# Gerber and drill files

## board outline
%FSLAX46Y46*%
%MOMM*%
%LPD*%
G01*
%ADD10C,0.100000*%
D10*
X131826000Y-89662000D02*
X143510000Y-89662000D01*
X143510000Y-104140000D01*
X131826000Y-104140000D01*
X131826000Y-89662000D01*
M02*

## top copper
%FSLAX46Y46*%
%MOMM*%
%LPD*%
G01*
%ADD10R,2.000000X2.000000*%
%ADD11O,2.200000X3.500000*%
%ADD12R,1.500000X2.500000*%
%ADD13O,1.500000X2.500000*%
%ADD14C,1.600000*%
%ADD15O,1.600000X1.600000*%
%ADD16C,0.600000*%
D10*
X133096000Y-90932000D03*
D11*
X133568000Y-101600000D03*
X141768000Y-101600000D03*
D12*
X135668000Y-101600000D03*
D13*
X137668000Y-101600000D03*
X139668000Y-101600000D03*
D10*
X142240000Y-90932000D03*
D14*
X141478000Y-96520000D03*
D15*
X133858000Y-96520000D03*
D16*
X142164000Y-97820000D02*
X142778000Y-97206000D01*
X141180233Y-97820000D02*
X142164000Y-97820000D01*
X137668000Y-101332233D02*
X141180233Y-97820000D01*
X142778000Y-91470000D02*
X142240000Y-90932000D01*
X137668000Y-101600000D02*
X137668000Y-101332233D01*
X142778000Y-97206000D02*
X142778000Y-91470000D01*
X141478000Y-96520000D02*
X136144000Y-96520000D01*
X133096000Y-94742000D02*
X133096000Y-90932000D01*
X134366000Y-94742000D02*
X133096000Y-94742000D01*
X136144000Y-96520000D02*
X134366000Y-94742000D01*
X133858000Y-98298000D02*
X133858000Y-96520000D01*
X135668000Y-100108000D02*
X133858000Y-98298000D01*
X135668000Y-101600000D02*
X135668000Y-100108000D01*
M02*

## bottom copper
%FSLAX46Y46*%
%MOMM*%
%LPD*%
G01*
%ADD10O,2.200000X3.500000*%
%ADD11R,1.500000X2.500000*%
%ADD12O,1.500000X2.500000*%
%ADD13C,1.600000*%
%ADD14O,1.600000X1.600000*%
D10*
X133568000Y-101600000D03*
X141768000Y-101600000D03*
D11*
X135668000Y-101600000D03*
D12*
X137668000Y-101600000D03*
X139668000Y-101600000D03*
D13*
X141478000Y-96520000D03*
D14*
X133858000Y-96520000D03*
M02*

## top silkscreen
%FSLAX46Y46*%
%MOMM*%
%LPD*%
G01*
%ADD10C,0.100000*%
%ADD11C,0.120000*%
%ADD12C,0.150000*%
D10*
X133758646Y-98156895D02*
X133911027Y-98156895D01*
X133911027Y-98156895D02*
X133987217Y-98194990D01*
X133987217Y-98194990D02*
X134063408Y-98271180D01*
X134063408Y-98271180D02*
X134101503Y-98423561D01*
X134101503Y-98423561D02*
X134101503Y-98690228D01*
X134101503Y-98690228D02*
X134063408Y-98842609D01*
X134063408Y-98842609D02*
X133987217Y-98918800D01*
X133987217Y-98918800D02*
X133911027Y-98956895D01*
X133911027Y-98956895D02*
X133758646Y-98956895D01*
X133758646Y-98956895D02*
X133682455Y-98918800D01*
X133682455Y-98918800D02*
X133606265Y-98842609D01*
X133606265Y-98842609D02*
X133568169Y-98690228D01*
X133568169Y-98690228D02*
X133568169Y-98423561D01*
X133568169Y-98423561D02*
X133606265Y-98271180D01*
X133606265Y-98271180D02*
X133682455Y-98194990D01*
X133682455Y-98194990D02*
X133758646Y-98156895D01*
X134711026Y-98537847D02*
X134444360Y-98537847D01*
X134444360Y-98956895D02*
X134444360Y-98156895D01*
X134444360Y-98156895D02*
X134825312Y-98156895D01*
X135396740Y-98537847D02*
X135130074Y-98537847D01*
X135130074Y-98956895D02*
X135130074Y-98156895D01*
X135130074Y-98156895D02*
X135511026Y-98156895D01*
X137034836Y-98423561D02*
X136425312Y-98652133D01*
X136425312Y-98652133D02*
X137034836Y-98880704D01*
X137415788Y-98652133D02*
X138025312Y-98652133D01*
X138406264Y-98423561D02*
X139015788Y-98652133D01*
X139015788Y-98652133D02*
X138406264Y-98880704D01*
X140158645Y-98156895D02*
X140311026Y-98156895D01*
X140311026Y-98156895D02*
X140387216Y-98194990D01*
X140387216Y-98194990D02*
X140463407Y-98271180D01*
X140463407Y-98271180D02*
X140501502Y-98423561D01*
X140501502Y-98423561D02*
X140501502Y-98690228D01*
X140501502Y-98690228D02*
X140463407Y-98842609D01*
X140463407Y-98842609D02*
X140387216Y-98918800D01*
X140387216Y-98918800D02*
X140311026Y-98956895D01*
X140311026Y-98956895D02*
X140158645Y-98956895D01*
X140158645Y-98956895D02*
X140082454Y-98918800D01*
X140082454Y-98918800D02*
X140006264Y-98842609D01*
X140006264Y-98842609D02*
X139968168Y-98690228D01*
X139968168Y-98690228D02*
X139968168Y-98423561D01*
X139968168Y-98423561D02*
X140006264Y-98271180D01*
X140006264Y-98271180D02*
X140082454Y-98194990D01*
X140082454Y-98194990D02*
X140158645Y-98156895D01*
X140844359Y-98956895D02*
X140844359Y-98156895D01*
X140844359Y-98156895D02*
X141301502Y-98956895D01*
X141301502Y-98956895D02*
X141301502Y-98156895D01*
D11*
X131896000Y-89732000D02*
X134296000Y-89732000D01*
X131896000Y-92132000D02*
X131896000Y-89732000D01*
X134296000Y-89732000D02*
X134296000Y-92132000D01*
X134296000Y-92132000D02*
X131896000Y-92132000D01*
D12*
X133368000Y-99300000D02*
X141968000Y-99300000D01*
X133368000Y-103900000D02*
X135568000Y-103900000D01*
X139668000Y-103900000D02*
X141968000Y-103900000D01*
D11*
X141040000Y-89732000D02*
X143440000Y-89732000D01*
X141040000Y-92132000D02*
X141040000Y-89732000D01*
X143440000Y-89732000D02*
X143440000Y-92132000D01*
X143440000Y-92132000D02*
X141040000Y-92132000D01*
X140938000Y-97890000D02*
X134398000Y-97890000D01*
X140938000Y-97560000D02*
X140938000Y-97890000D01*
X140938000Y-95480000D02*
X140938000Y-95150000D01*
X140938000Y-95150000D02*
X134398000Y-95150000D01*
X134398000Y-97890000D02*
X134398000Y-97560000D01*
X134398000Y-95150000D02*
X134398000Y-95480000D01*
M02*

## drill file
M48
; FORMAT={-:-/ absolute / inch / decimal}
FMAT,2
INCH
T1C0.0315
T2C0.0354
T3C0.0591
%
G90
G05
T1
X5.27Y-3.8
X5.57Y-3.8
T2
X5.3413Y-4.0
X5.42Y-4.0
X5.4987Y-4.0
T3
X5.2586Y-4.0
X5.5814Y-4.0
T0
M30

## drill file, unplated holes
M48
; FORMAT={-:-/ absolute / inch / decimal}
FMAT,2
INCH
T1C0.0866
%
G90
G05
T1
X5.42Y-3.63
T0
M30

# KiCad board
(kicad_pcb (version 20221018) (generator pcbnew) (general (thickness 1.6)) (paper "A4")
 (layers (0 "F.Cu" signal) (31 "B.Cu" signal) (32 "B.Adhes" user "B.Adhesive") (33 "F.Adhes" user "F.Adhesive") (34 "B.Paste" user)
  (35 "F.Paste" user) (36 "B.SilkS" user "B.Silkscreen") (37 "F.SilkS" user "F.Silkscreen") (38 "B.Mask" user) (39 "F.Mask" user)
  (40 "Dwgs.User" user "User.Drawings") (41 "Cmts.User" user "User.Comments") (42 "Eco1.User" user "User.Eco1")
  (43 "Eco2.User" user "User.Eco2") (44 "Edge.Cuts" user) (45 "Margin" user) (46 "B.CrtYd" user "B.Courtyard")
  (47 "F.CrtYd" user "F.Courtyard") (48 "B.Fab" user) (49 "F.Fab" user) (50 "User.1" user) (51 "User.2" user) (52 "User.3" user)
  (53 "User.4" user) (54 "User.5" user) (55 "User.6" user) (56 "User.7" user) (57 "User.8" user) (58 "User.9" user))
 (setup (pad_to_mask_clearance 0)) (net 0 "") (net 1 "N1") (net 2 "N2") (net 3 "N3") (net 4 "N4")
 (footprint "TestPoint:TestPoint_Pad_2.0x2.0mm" (layer "F.Cu") (at 133.096 90.932)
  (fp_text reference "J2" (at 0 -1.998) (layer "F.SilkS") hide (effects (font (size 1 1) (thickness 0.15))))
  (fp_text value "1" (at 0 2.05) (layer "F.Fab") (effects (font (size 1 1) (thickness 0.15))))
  (fp_line (start -1.2 -1.2) (end 1.2 -1.2) (stroke (width 0.12) (type solid)) (layer "F.SilkS"))
  (fp_line (start -1.2 1.2) (end -1.2 -1.2) (stroke (width 0.12) (type solid)) (layer "F.SilkS"))
  (fp_line (start 1.2 -1.2) (end 1.2 1.2) (stroke (width 0.12) (type solid)) (layer "F.SilkS"))
  (fp_line (start 1.2 1.2) (end -1.2 1.2) (stroke (width 0.12) (type solid)) (layer "F.SilkS"))
  (pad "1" smd rect (at 0 0) (size 2 2) (layers "F.Cu" "F.Mask") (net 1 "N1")))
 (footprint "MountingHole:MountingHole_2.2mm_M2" (layer "F.Cu") (at 137.668 92.202)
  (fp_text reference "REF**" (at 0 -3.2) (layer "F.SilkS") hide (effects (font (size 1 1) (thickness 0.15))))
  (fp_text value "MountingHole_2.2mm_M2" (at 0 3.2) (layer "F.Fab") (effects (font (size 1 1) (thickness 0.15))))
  (pad "" np_thru_hole circle (at 0 0) (size 2.2 2.2) (drill 2.2) (layers "*.Cu" "*.Mask")))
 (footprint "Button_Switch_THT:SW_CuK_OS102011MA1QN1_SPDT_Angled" (layer "F.Cu") (at 135.668 101.6)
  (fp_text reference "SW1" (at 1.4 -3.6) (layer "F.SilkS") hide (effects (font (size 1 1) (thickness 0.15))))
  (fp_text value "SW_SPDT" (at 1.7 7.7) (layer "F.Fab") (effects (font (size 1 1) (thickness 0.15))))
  (fp_line (start -2.3 -2.3) (end 6.3 -2.3) (stroke (width 0.15) (type solid)) (layer "F.SilkS"))
  (fp_line (start -2.3 2.3) (end -0.1 2.3) (stroke (width 0.15) (type solid)) (layer "F.SilkS"))
  (fp_line (start 4 2.3) (end 6.3 2.3) (stroke (width 0.15) (type solid)) (layer "F.SilkS"))
  (pad "" thru_hole oval (at -2.1 0) (size 2.2 3.5) (drill 1.5) (layers "*.Cu" "*.Mask"))
  (pad "" thru_hole oval (at 6.1 0) (size 2.2 3.5) (drill 1.5) (layers "*.Cu" "*.Mask"))
  (pad "1" thru_hole rect (at 0 0) (size 1.5 2.5) (drill 0.9) (layers "*.Cu" "*.Mask") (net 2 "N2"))
  (pad "2" thru_hole oval (at 2 0) (size 1.5 2.5) (drill 0.9) (layers "*.Cu" "*.Mask") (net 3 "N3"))
  (pad "3" thru_hole oval (at 4 0) (size 1.5 2.5) (drill 0.9) (layers "*.Cu" "*.Mask") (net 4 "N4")))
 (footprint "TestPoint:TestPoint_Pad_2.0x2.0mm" (layer "F.Cu") (at 142.24 90.932)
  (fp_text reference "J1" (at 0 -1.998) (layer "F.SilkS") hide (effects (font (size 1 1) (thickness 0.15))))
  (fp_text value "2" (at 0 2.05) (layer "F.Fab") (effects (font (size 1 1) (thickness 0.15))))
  (fp_line (start -1.2 -1.2) (end 1.2 -1.2) (stroke (width 0.12) (type solid)) (layer "F.SilkS"))
  (fp_line (start -1.2 1.2) (end -1.2 -1.2) (stroke (width 0.12) (type solid)) (layer "F.SilkS"))
  (fp_line (start 1.2 -1.2) (end 1.2 1.2) (stroke (width 0.12) (type solid)) (layer "F.SilkS"))
  (fp_line (start 1.2 1.2) (end -1.2 1.2) (stroke (width 0.12) (type solid)) (layer "F.SilkS"))
  (pad "1" smd rect (at 0 0) (size 2 2) (layers "F.Cu" "F.Mask") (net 3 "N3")))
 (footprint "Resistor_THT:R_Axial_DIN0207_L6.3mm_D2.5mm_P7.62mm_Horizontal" (layer "F.Cu") (at 141.478 96.52 180)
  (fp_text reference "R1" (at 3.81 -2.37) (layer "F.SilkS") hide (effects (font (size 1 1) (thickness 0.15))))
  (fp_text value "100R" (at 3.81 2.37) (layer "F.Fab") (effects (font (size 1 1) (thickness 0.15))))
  (fp_line (start 0.54 -1.37) (end 7.08 -1.37) (stroke (width 0.12) (type solid)) (layer "F.SilkS"))
  (fp_line (start 0.54 -1.04) (end 0.54 -1.37) (stroke (width 0.12) (type solid)) (layer "F.SilkS"))
  (fp_line (start 0.54 1.04) (end 0.54 1.37) (stroke (width 0.12) (type solid)) (layer "F.SilkS"))
  (fp_line (start 0.54 1.37) (end 7.08 1.37) (stroke (width 0.12) (type solid)) (layer "F.SilkS"))
  (fp_line (start 7.08 -1.37) (end 7.08 -1.04) (stroke (width 0.12) (type solid)) (layer "F.SilkS"))
  (fp_line (start 7.08 1.37) (end 7.08 1.04) (stroke (width 0.12) (type solid)) (layer "F.SilkS"))
  (pad "1" thru_hole circle (at 0 0 180) (size 1.6 1.6) (drill 0.8) (layers "*.Cu" "*.Mask") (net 1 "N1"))
  (pad "2" thru_hole oval (at 7.62 0 180) (size 1.6 1.6) (drill 0.8) (layers "*.Cu" "*.Mask") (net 2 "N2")))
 (gr_rect (start 131.826 89.662) (end 143.51 104.14) (stroke (width 0.1) (type default)) (fill none) (layer "Edge.Cuts"))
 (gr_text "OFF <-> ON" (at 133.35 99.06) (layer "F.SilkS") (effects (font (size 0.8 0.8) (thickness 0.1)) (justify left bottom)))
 (segment (start 142.164 97.82) (end 142.778 97.206) (width 0.6) (layer "F.Cu") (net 3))
 (segment (start 141.180233 97.82) (end 142.164 97.82) (width 0.6) (layer "F.Cu") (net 3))
 (segment (start 137.668 101.332233) (end 141.180233 97.82) (width 0.6) (layer "F.Cu") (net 3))
 (segment (start 142.778 91.47) (end 142.24 90.932) (width 0.6) (layer "F.Cu") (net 3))
 (segment (start 137.668 101.6) (end 137.668 101.332233) (width 0.6) (layer "F.Cu") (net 3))
 (segment (start 142.778 97.206) (end 142.778 91.47) (width 0.6) (layer "F.Cu") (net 3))
 (segment (start 141.478 96.52) (end 136.144 96.52) (width 0.6) (layer "F.Cu") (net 1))
 (segment (start 133.096 94.742) (end 133.096 90.932) (width 0.6) (layer "F.Cu") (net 1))
 (segment (start 134.366 94.742) (end 133.096 94.742) (width 0.6) (layer "F.Cu") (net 1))
 (segment (start 136.144 96.52) (end 134.366 94.742) (width 0.6) (layer "F.Cu") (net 1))
 (segment (start 133.858 98.298) (end 133.858 96.52) (width 0.6) (layer "F.Cu") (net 2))
 (segment (start 135.668 100.108) (end 133.858 98.298) (width 0.6) (layer "F.Cu") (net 2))
 (segment (start 135.668 101.6) (end 135.668 100.108) (width 0.6) (layer "F.Cu") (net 2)))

